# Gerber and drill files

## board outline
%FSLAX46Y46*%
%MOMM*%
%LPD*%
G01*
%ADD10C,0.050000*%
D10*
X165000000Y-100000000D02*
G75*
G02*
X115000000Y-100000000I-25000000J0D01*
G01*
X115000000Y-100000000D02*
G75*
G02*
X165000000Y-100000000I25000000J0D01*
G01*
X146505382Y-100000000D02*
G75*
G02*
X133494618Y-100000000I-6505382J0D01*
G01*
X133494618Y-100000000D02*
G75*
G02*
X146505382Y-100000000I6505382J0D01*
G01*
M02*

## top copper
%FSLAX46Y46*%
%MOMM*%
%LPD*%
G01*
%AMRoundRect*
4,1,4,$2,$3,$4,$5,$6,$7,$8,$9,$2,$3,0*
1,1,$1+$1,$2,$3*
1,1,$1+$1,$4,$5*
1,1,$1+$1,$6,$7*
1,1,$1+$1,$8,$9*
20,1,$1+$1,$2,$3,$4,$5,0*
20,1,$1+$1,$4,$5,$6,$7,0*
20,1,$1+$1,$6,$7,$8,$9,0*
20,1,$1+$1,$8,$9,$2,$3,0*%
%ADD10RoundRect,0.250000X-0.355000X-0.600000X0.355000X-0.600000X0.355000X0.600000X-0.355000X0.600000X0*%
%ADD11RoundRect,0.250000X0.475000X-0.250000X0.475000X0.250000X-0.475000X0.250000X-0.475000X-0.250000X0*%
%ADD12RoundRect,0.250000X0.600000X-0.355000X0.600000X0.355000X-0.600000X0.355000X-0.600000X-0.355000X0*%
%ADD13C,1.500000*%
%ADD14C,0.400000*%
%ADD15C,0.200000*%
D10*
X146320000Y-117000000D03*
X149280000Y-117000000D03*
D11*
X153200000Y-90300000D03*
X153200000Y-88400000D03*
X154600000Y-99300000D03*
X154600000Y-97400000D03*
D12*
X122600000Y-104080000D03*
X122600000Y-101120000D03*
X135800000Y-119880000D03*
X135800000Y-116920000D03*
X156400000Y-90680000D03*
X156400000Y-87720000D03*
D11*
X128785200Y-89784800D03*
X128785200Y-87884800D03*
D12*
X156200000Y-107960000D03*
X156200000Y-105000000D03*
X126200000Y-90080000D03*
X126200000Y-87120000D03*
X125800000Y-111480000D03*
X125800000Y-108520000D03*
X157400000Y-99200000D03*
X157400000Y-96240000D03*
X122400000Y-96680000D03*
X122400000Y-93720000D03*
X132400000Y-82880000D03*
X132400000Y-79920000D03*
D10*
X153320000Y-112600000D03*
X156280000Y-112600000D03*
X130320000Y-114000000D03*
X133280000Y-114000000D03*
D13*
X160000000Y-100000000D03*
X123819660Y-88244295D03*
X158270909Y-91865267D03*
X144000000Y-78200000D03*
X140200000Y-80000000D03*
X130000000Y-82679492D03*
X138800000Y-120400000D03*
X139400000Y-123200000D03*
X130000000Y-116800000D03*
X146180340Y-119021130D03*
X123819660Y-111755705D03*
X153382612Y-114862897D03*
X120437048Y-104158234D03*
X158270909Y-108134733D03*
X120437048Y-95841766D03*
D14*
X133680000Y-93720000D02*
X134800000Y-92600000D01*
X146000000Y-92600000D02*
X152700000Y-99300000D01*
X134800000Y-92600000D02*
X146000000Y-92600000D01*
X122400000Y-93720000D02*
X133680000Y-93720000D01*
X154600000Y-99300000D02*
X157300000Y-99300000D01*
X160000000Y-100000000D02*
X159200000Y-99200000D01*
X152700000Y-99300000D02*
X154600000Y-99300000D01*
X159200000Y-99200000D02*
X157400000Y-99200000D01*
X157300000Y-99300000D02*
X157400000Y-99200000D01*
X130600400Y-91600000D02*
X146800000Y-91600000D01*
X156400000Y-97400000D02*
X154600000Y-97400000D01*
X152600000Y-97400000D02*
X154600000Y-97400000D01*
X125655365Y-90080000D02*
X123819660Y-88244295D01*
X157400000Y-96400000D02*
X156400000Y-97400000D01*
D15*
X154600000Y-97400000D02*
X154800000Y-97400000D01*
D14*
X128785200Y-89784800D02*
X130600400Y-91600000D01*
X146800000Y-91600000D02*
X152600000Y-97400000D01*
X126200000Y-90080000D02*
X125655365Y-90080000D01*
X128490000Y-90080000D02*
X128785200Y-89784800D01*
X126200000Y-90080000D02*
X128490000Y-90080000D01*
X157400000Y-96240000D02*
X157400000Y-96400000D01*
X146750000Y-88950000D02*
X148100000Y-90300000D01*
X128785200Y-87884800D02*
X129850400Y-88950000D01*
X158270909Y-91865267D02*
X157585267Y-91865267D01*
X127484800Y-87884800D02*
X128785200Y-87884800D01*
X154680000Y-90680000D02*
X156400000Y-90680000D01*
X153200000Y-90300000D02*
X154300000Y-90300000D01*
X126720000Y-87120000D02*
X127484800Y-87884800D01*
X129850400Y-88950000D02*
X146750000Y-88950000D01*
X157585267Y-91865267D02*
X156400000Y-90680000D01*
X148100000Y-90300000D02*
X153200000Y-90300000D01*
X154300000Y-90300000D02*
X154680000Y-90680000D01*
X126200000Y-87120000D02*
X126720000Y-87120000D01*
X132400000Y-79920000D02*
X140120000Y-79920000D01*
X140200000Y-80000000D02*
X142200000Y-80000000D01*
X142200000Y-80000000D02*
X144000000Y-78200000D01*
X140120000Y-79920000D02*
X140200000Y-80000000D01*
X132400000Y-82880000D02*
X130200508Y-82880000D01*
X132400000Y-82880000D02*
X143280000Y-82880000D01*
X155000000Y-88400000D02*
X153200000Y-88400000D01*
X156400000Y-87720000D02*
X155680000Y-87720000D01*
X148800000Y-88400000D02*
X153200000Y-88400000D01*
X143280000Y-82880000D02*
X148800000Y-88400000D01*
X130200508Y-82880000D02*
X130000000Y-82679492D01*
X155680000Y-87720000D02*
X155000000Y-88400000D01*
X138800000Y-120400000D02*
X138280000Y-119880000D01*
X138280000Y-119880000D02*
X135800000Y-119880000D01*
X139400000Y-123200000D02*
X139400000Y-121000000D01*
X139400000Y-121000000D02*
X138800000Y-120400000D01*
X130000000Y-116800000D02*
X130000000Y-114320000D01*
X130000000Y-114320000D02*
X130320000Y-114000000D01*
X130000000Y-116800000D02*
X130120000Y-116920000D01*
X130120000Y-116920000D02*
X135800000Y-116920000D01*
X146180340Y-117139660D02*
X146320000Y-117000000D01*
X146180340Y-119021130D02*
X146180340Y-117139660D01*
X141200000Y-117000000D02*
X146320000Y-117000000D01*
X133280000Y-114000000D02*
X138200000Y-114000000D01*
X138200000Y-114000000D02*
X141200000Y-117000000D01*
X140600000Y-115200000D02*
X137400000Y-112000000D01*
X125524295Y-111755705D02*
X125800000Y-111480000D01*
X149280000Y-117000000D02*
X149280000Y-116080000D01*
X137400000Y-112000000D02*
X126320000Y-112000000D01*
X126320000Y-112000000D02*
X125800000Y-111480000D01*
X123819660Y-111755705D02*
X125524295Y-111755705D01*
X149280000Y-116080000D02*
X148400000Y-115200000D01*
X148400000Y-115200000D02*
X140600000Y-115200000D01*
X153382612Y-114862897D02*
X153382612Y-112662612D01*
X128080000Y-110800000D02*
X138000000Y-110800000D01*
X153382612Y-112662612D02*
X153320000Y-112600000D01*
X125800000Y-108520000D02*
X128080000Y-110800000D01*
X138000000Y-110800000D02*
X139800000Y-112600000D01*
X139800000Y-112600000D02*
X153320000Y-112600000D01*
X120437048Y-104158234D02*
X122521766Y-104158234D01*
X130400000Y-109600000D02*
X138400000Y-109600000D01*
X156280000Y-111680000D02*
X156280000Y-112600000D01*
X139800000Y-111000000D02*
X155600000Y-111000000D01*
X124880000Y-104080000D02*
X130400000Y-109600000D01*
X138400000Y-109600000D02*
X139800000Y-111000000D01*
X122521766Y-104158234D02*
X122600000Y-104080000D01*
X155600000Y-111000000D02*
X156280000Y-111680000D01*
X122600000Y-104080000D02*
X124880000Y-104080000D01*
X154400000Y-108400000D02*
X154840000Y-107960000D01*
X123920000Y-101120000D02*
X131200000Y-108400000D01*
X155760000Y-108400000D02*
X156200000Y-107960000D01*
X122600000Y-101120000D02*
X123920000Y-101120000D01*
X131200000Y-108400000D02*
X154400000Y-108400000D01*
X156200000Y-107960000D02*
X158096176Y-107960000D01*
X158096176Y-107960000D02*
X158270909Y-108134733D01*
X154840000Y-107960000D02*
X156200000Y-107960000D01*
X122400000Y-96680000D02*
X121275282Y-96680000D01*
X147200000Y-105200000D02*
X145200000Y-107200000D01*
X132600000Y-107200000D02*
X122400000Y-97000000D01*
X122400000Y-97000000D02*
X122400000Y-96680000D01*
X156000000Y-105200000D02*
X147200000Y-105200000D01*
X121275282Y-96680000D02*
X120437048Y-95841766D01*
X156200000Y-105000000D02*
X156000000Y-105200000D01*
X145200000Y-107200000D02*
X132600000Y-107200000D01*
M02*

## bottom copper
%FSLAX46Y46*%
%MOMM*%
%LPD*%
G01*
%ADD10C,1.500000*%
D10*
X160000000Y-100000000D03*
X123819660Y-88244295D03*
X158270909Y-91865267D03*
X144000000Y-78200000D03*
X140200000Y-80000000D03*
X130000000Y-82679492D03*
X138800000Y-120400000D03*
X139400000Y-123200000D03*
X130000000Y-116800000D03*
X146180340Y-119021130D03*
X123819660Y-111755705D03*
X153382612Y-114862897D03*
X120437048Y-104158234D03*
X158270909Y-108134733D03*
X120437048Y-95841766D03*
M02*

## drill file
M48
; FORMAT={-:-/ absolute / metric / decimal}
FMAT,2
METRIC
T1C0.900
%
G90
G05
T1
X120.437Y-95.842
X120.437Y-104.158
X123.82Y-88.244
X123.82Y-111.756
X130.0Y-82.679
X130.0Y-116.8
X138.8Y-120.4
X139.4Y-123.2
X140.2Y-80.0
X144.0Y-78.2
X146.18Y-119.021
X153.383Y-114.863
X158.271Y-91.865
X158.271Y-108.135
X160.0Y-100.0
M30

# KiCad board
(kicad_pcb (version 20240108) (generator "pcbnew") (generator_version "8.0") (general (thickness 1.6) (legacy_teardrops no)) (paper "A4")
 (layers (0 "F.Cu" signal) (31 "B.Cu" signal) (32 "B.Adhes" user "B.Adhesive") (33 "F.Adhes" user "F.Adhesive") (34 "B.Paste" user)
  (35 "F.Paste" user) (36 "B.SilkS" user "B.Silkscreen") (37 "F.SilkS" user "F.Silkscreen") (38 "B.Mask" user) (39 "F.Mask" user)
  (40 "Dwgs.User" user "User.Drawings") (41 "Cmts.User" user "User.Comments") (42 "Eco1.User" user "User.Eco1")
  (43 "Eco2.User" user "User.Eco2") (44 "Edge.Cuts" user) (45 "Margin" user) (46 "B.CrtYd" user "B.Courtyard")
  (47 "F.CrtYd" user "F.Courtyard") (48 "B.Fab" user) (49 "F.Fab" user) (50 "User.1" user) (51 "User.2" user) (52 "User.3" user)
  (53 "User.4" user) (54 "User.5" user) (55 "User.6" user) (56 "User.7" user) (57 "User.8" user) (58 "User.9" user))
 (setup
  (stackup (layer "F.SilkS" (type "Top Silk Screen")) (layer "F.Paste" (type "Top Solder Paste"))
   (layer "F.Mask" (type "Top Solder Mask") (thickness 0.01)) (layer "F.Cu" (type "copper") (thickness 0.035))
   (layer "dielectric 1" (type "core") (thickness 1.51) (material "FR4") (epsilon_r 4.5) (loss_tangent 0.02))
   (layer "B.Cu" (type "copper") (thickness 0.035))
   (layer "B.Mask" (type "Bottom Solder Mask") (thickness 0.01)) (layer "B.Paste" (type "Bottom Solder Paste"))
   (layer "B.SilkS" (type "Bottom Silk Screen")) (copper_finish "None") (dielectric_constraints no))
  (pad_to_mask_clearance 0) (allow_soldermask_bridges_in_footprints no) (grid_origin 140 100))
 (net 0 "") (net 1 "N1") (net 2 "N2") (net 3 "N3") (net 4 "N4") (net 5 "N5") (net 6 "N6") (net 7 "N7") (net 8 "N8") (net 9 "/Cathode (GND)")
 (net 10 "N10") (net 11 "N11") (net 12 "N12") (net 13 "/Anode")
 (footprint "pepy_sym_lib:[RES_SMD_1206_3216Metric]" (layer "F.Cu") (at 147.8 117)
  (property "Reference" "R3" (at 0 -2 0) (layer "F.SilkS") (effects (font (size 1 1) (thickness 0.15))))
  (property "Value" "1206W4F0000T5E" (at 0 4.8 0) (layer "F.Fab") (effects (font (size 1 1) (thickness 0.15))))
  (pad "1" smd roundrect (at -1.48 0) (size 1.21 1.7) (layers "F.Cu" "F.Paste" "F.Mask") (roundrect_rratio 0.2066115702) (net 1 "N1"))
  (pad "2" smd roundrect (at 1.48 0) (size 1.21 1.7) (layers "F.Cu" "F.Paste" "F.Mask") (roundrect_rratio 0.2066115702) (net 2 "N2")))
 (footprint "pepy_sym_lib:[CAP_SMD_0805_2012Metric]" (layer "F.Cu") (at 153.2148 89.3152 90)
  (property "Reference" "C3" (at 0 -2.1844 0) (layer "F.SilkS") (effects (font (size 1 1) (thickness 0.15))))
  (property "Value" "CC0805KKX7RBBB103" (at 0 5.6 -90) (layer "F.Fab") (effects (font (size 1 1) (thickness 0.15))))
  (pad "1" smd roundrect (at -0.9848 -0.0148 90) (size 1 1.45) (layers "F.Cu" "F.Paste" "F.Mask") (roundrect_rratio 0.25) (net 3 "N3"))
  (pad "2" smd roundrect (at 0.9152 -0.0148 90) (size 1 1.45) (layers "F.Cu" "F.Paste" "F.Mask") (roundrect_rratio 0.25) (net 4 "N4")))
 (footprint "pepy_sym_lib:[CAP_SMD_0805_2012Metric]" (layer "F.Cu") (at 154.6148 98.3152 90)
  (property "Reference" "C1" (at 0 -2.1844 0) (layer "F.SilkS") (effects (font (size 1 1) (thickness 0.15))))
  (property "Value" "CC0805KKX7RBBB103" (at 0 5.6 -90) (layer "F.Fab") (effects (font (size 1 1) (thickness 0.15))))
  (pad "1" smd roundrect (at -0.9848 -0.0148 90) (size 1 1.45) (layers "F.Cu" "F.Paste" "F.Mask") (roundrect_rratio 0.25) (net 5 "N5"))
  (pad "2" smd roundrect (at 0.9152 -0.0148 90) (size 1 1.45) (layers "F.Cu" "F.Paste" "F.Mask") (roundrect_rratio 0.25) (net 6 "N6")))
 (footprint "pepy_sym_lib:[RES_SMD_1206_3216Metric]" (layer "F.Cu") (at 122.6 102.6 90)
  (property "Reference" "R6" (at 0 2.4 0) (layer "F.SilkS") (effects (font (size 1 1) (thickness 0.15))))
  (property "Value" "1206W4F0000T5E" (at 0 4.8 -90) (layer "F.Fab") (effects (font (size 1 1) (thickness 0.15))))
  (pad "1" smd roundrect (at -1.48 0 90) (size 1.21 1.7) (layers "F.Cu" "F.Paste" "F.Mask") (roundrect_rratio 0.2066115702) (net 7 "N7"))
  (pad "2" smd roundrect (at 1.48 0 90) (size 1.21 1.7) (layers "F.Cu" "F.Paste" "F.Mask") (roundrect_rratio 0.2066115702) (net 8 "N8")))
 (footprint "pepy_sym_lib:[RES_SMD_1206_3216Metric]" (layer "F.Cu") (at 135.8 118.4 90)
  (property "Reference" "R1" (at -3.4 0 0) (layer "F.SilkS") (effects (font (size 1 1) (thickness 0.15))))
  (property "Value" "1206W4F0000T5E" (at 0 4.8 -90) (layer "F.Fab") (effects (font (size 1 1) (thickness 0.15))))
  (pad "1" smd roundrect (at -1.48 0 90) (size 1.21 1.7) (layers "F.Cu" "F.Paste" "F.Mask") (roundrect_rratio 0.2066115702)
   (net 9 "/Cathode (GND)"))
  (pad "2" smd roundrect (at 1.48 0 90) (size 1.21 1.7) (layers "F.Cu" "F.Paste" "F.Mask") (roundrect_rratio 0.2066115702) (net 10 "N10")))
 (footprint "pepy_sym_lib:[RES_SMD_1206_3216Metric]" (layer "F.Cu") (at 156.4 89.2 90)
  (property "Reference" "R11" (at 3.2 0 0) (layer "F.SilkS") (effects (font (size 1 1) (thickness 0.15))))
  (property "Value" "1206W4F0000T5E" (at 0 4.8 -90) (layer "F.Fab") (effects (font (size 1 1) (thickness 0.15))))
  (pad "1" smd roundrect (at -1.48 0 90) (size 1.21 1.7) (layers "F.Cu" "F.Paste" "F.Mask") (roundrect_rratio 0.2066115702) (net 3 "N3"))
  (pad "2" smd roundrect (at 1.48 0 90) (size 1.21 1.7) (layers "F.Cu" "F.Paste" "F.Mask") (roundrect_rratio 0.2066115702) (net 4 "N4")))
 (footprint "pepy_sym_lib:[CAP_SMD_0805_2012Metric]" (layer "F.Cu") (at 128.8 88.8 90)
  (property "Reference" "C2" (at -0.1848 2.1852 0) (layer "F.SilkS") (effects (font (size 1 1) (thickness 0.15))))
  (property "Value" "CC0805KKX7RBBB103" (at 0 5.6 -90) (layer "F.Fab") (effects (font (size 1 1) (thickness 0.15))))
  (pad "1" smd roundrect (at -0.9848 -0.0148 90) (size 1 1.45) (layers "F.Cu" "F.Paste" "F.Mask") (roundrect_rratio 0.25) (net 6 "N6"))
  (pad "2" smd roundrect (at 0.9152 -0.0148 90) (size 1 1.45) (layers "F.Cu" "F.Paste" "F.Mask") (roundrect_rratio 0.25) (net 3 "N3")))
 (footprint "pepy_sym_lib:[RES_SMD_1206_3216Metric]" (layer "F.Cu") (at 156.2 106.48 90)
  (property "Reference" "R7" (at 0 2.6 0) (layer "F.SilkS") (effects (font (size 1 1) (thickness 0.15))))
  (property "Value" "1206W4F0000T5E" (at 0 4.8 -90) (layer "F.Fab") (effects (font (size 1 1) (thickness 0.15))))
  (pad "1" smd roundrect (at -1.48 0 90) (size 1.21 1.7) (layers "F.Cu" "F.Paste" "F.Mask") (roundrect_rratio 0.2066115702) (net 8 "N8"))
  (pad "2" smd roundrect (at 1.48 0 90) (size 1.21 1.7) (layers "F.Cu" "F.Paste" "F.Mask") (roundrect_rratio 0.2066115702) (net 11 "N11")))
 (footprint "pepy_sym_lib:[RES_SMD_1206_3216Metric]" (layer "F.Cu") (at 126.2 88.6 90)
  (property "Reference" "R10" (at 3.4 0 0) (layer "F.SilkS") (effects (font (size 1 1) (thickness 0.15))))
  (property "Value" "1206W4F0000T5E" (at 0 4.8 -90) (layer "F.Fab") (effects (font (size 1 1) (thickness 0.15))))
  (pad "1" smd roundrect (at -1.48 0 90) (size 1.21 1.7) (layers "F.Cu" "F.Paste" "F.Mask") (roundrect_rratio 0.2066115702) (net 6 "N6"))
  (pad "2" smd roundrect (at 1.48 0 90) (size 1.21 1.7) (layers "F.Cu" "F.Paste" "F.Mask") (roundrect_rratio 0.2066115702) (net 3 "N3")))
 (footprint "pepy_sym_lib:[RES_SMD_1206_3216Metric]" (layer "F.Cu") (at 125.8 110 90)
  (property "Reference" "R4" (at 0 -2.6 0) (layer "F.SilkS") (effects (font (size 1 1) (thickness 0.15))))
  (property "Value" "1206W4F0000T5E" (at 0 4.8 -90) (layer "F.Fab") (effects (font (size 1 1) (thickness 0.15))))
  (pad "1" smd roundrect (at -1.48 0 90) (size 1.21 1.7) (layers "F.Cu" "F.Paste" "F.Mask") (roundrect_rratio 0.2066115702) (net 2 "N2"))
  (pad "2" smd roundrect (at 1.48 0 90) (size 1.21 1.7) (layers "F.Cu" "F.Paste" "F.Mask") (roundrect_rratio 0.2066115702) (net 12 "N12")))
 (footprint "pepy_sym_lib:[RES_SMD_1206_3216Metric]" (layer "F.Cu") (at 157.4 97.72 90)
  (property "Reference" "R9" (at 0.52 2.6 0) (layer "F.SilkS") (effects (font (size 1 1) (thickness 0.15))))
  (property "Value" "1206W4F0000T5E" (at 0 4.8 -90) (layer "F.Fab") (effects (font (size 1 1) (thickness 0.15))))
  (pad "1" smd roundrect (at -1.48 0 90) (size 1.21 1.7) (layers "F.Cu" "F.Paste" "F.Mask") (roundrect_rratio 0.2066115702) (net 5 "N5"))
  (pad "2" smd roundrect (at 1.48 0 90) (size 1.21 1.7) (layers "F.Cu" "F.Paste" "F.Mask") (roundrect_rratio 0.2066115702) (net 6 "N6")))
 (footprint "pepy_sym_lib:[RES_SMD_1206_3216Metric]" (layer "F.Cu") (at 122.4 95.2 90)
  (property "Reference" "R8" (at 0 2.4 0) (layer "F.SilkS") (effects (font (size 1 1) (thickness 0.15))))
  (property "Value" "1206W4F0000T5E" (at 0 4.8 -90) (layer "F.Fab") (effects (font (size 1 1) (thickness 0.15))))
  (pad "1" smd roundrect (at -1.48 0 90) (size 1.21 1.7) (layers "F.Cu" "F.Paste" "F.Mask") (roundrect_rratio 0.2066115702) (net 11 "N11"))
  (pad "2" smd roundrect (at 1.48 0 90) (size 1.21 1.7) (layers "F.Cu" "F.Paste" "F.Mask") (roundrect_rratio 0.2066115702) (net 5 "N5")))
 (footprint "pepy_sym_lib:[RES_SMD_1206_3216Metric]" (layer "F.Cu") (at 132.4 81.4 90)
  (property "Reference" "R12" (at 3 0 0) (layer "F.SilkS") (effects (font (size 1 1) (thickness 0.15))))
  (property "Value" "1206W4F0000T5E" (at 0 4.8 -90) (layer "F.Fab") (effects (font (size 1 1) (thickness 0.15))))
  (pad "1" smd roundrect (at -1.48 0 90) (size 1.21 1.7) (layers "F.Cu" "F.Paste" "F.Mask") (roundrect_rratio 0.2066115702) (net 4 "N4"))
  (pad "2" smd roundrect (at 1.48 0 90) (size 1.21 1.7) (layers "F.Cu" "F.Paste" "F.Mask") (roundrect_rratio 0.2066115702) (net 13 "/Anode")))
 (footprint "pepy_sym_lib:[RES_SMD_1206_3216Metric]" (layer "F.Cu") (at 154.8 112.6)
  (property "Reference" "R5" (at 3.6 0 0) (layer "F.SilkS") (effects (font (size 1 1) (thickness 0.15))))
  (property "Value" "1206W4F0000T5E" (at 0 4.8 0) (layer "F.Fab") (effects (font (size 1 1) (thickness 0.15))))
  (pad "1" smd roundrect (at -1.48 0) (size 1.21 1.7) (layers "F.Cu" "F.Paste" "F.Mask") (roundrect_rratio 0.2066115702) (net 12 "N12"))
  (pad "2" smd roundrect (at 1.48 0) (size 1.21 1.7) (layers "F.Cu" "F.Paste" "F.Mask") (roundrect_rratio 0.2066115702) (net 7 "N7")))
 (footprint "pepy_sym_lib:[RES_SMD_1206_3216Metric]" (layer "F.Cu") (at 131.8 114)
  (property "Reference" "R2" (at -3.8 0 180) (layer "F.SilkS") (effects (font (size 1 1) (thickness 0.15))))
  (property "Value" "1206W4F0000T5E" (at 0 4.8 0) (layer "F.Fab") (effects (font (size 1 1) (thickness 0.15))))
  (pad "1" smd roundrect (at -1.48 0) (size 1.21 1.7) (layers "F.Cu" "F.Paste" "F.Mask") (roundrect_rratio 0.2066115702) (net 10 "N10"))
  (pad "2" smd roundrect (at 1.48 0) (size 1.21 1.7) (layers "F.Cu" "F.Paste" "F.Mask") (roundrect_rratio 0.2066115702) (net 1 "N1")))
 (gr_circle (center 140 100) (end 165 100) (stroke (width 0.05) (type default)) (fill none) (layer "Edge.Cuts"))
 (gr_circle (center 140 100) (end 144.6 104.6) (stroke (width 0.05) (type default)) (fill none) (layer "Edge.Cuts"))
 (segment (start 133.68 93.72) (end 134.8 92.6) (width 0.4) (layer "F.Cu") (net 5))
 (segment (start 146 92.6) (end 152.7 99.3) (width 0.4) (layer "F.Cu") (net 5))
 (segment (start 134.8 92.6) (end 146 92.6) (width 0.4) (layer "F.Cu") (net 5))
 (segment (start 122.4 93.72) (end 133.68 93.72) (width 0.4) (layer "F.Cu") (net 5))
 (segment (start 154.6 99.3) (end 157.3 99.3) (width 0.4) (layer "F.Cu") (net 5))
 (segment (start 160 100) (end 159.2 99.2) (width 0.4) (layer "F.Cu") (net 5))
 (segment (start 152.7 99.3) (end 154.6 99.3) (width 0.4) (layer "F.Cu") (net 5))
 (segment (start 159.2 99.2) (end 157.4 99.2) (width 0.4) (layer "F.Cu") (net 5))
 (segment (start 157.3 99.3) (end 157.4 99.2) (width 0.4) (layer "F.Cu") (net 5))
 (via (at 160 100) (size 1.5) (drill 0.9) (layers "F.Cu" "B.Cu") (free yes) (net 5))
 (segment (start 130.6004 91.6) (end 146.8 91.6) (width 0.4) (layer "F.Cu") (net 6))
 (segment (start 156.4 97.4) (end 154.6 97.4) (width 0.4) (layer "F.Cu") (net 6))
 (segment (start 152.6 97.4) (end 154.6 97.4) (width 0.4) (layer "F.Cu") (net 6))
 (segment (start 125.655365 90.08) (end 123.81966 88.244295) (width 0.4) (layer "F.Cu") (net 6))
 (segment (start 157.4 96.4) (end 156.4 97.4) (width 0.4) (layer "F.Cu") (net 6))
 (segment (start 154.6 97.4) (end 154.8 97.4) (width 0.2) (layer "F.Cu") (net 6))
 (segment (start 128.7852 89.7848) (end 130.6004 91.6) (width 0.4) (layer "F.Cu") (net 6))
 (segment (start 146.8 91.6) (end 152.6 97.4) (width 0.4) (layer "F.Cu") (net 6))
 (segment (start 126.2 90.08) (end 125.655365 90.08) (width 0.4) (layer "F.Cu") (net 6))
 (segment (start 128.49 90.08) (end 128.7852 89.7848) (width 0.4) (layer "F.Cu") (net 6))
 (segment (start 126.2 90.08) (end 128.49 90.08) (width 0.4) (layer "F.Cu") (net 6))
 (segment (start 157.4 96.24) (end 157.4 96.4) (width 0.4) (layer "F.Cu") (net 6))
 (via (at 123.81966 88.244295) (size 1.5) (drill 0.9) (layers "F.Cu" "B.Cu") (free yes) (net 6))
 (segment (start 146.75 88.95) (end 148.1 90.3) (width 0.4) (layer "F.Cu") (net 3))
 (segment (start 128.7852 87.8848) (end 129.8504 88.95) (width 0.4) (layer "F.Cu") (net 3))
 (segment (start 158.270909 91.865267) (end 157.585267 91.865267) (width 0.4) (layer "F.Cu") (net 3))
 (segment (start 127.4848 87.8848) (end 128.7852 87.8848) (width 0.4) (layer "F.Cu") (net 3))
 (segment (start 154.68 90.68) (end 156.4 90.68) (width 0.4) (layer "F.Cu") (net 3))
 (segment (start 153.2 90.3) (end 154.3 90.3) (width 0.4) (layer "F.Cu") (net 3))
 (segment (start 126.72 87.12) (end 127.4848 87.8848) (width 0.4) (layer "F.Cu") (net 3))
 (segment (start 129.8504 88.95) (end 146.75 88.95) (width 0.4) (layer "F.Cu") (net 3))
 (segment (start 157.585267 91.865267) (end 156.4 90.68) (width 0.4) (layer "F.Cu") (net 3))
 (segment (start 148.1 90.3) (end 153.2 90.3) (width 0.4) (layer "F.Cu") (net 3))
 (segment (start 154.3 90.3) (end 154.68 90.68) (width 0.4) (layer "F.Cu") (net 3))
 (segment (start 126.2 87.12) (end 126.72 87.12) (width 0.4) (layer "F.Cu") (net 3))
 (via (at 158.270909 91.865267) (size 1.5) (drill 0.9) (layers "F.Cu" "B.Cu") (free yes) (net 3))
 (segment (start 132.4 79.92) (end 140.12 79.92) (width 0.4) (layer "F.Cu") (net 13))
 (segment (start 140.2 80) (end 142.2 80) (width 0.4) (layer "F.Cu") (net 13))
 (segment (start 142.2 80) (end 144 78.2) (width 0.4) (layer "F.Cu") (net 13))
 (segment (start 140.12 79.92) (end 140.2 80) (width 0.4) (layer "F.Cu") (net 13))
 (via (at 144 78.2) (size 1.5) (drill 0.9) (layers "F.Cu" "B.Cu") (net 13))
 (via (at 140.2 80) (size 1.5) (drill 0.9) (layers "F.Cu" "B.Cu") (free yes) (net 13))
 (segment (start 132.4 82.88) (end 130.200508 82.88) (width 0.4) (layer "F.Cu") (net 4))
 (segment (start 132.4 82.88) (end 143.28 82.88) (width 0.4) (layer "F.Cu") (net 4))
 (segment (start 155 88.4) (end 153.2 88.4) (width 0.4) (layer "F.Cu") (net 4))
 (segment (start 156.4 87.72) (end 155.68 87.72) (width 0.4) (layer "F.Cu") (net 4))
 (segment (start 148.8 88.4) (end 153.2 88.4) (width 0.4) (layer "F.Cu") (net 4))
 (segment (start 143.28 82.88) (end 148.8 88.4) (width 0.4) (layer "F.Cu") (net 4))
 (segment (start 130.200508 82.88) (end 130 82.679492) (width 0.4) (layer "F.Cu") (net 4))
 (segment (start 155.68 87.72) (end 155 88.4) (width 0.4) (layer "F.Cu") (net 4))
 (via (at 130 82.679492) (size 1.5) (drill 0.9) (layers "F.Cu" "B.Cu") (free yes) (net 4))
 (segment (start 138.8 120.4) (end 138.28 119.88) (width 0.4) (layer "F.Cu") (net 9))
 (segment (start 138.28 119.88) (end 135.8 119.88) (width 0.4) (layer "F.Cu") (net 9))
 (segment (start 139.4 123.2) (end 139.4 121) (width 0.4) (layer "F.Cu") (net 9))
 (segment (start 139.4 121) (end 138.8 120.4) (width 0.4) (layer "F.Cu") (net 9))
 (via (at 138.8 120.4) (size 1.5) (drill 0.9) (layers "F.Cu" "B.Cu") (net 9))
 (via (at 139.4 123.2) (size 1.5) (drill 0.9) (layers "F.Cu" "B.Cu") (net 9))
 (segment (start 130 116.8) (end 130 114.32) (width 0.4) (layer "F.Cu") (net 10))
 (segment (start 130 114.32) (end 130.32 114) (width 0.4) (layer "F.Cu") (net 10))
 (segment (start 130 116.8) (end 130.12 116.92) (width 0.4) (layer "F.Cu") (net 10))
 (segment (start 130.12 116.92) (end 135.8 116.92) (width 0.4) (layer "F.Cu") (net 10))
 (via (at 130 116.8) (size 1.5) (drill 0.9) (layers "F.Cu" "B.Cu") (free yes) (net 10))
 (segment (start 146.18034 117.13966) (end 146.32 117) (width 0.4) (layer "F.Cu") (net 1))
 (segment (start 146.18034 119.02113) (end 146.18034 117.13966) (width 0.4) (layer "F.Cu") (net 1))
 (segment (start 141.2 117) (end 146.32 117) (width 0.4) (layer "F.Cu") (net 1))
 (segment (start 133.28 114) (end 138.2 114) (width 0.4) (layer "F.Cu") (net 1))
 (segment (start 138.2 114) (end 141.2 117) (width 0.4) (layer "F.Cu") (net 1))
 (via (at 146.18034 119.02113) (size 1.5) (drill 0.9) (layers "F.Cu" "B.Cu") (free yes) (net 1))
 (segment (start 140.6 115.2) (end 137.4 112) (width 0.4) (layer "F.Cu") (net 2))
 (segment (start 125.524295 111.755705) (end 125.8 111.48) (width 0.4) (layer "F.Cu") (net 2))
 (segment (start 149.28 117) (end 149.28 116.08) (width 0.4) (layer "F.Cu") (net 2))
 (segment (start 137.4 112) (end 126.32 112) (width 0.4) (layer "F.Cu") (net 2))
 (segment (start 126.32 112) (end 125.8 111.48) (width 0.4) (layer "F.Cu") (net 2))
 (segment (start 123.81966 111.755705) (end 125.524295 111.755705) (width 0.4) (layer "F.Cu") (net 2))
 (segment (start 149.28 116.08) (end 148.4 115.2) (width 0.4) (layer "F.Cu") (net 2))
 (segment (start 148.4 115.2) (end 140.6 115.2) (width 0.4) (layer "F.Cu") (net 2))
 (via (at 123.81966 111.755705) (size 1.5) (drill 0.9) (layers "F.Cu" "B.Cu") (free yes) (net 2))
 (segment (start 153.382612 114.862897) (end 153.382612 112.662612) (width 0.4) (layer "F.Cu") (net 12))
 (segment (start 128.08 110.8) (end 138 110.8) (width 0.4) (layer "F.Cu") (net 12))
 (segment (start 153.382612 112.662612) (end 153.32 112.6) (width 0.4) (layer "F.Cu") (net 12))
 (segment (start 125.8 108.52) (end 128.08 110.8) (width 0.4) (layer "F.Cu") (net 12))
 (segment (start 138 110.8) (end 139.8 112.6) (width 0.4) (layer "F.Cu") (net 12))
 (segment (start 139.8 112.6) (end 153.32 112.6) (width 0.4) (layer "F.Cu") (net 12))
 (via (at 153.382612 114.862897) (size 1.5) (drill 0.9) (layers "F.Cu" "B.Cu") (free yes) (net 12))
 (segment (start 120.437048 104.158234) (end 122.521766 104.158234) (width 0.4) (layer "F.Cu") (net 7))
 (segment (start 130.4 109.6) (end 138.4 109.6) (width 0.4) (layer "F.Cu") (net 7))
 (segment (start 156.28 111.68) (end 156.28 112.6) (width 0.4) (layer "F.Cu") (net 7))
 (segment (start 139.8 111) (end 155.6 111) (width 0.4) (layer "F.Cu") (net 7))
 (segment (start 124.88 104.08) (end 130.4 109.6) (width 0.4) (layer "F.Cu") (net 7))
 (segment (start 138.4 109.6) (end 139.8 111) (width 0.4) (layer "F.Cu") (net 7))
 (segment (start 122.521766 104.158234) (end 122.6 104.08) (width 0.4) (layer "F.Cu") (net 7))
 (segment (start 155.6 111) (end 156.28 111.68) (width 0.4) (layer "F.Cu") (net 7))
 (segment (start 122.6 104.08) (end 124.88 104.08) (width 0.4) (layer "F.Cu") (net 7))
 (via (at 120.437048 104.158234) (size 1.5) (drill 0.9) (layers "F.Cu" "B.Cu") (free yes) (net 7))
 (segment (start 154.4 108.4) (end 154.84 107.96) (width 0.4) (layer "F.Cu") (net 8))
 (segment (start 123.92 101.12) (end 131.2 108.4) (width 0.4) (layer "F.Cu") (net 8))
 (segment (start 155.76 108.4) (end 156.2 107.96) (width 0.4) (layer "F.Cu") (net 8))
 (segment (start 122.6 101.12) (end 123.92 101.12) (width 0.4) (layer "F.Cu") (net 8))
 (segment (start 131.2 108.4) (end 154.4 108.4) (width 0.4) (layer "F.Cu") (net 8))
 (segment (start 156.2 107.96) (end 158.096176 107.96) (width 0.4) (layer "F.Cu") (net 8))
 (segment (start 158.096176 107.96) (end 158.270909 108.134733) (width 0.4) (layer "F.Cu") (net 8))
 (segment (start 154.84 107.96) (end 156.2 107.96) (width 0.4) (layer "F.Cu") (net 8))
 (via (at 158.270909 108.134733) (size 1.5) (drill 0.9) (layers "F.Cu" "B.Cu") (free yes) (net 8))
 (segment (start 122.4 96.68) (end 121.275282 96.68) (width 0.4) (layer "F.Cu") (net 11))
 (segment (start 147.2 105.2) (end 145.2 107.2) (width 0.4) (layer "F.Cu") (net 11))
 (segment (start 132.6 107.2) (end 122.4 97) (width 0.4) (layer "F.Cu") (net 11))
 (segment (start 122.4 97) (end 122.4 96.68) (width 0.4) (layer "F.Cu") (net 11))
 (segment (start 156 105.2) (end 147.2 105.2) (width 0.4) (layer "F.Cu") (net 11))
 (segment (start 121.275282 96.68) (end 120.437048 95.841766) (width 0.4) (layer "F.Cu") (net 11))
 (segment (start 156.2 105) (end 156 105.2) (width 0.4) (layer "F.Cu") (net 11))
 (segment (start 145.2 107.2) (end 132.6 107.2) (width 0.4) (layer "F.Cu") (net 11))
 (via (at 120.437048 95.841766) (size 1.5) (drill 0.9) (layers "F.Cu" "B.Cu") (free yes) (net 11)))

